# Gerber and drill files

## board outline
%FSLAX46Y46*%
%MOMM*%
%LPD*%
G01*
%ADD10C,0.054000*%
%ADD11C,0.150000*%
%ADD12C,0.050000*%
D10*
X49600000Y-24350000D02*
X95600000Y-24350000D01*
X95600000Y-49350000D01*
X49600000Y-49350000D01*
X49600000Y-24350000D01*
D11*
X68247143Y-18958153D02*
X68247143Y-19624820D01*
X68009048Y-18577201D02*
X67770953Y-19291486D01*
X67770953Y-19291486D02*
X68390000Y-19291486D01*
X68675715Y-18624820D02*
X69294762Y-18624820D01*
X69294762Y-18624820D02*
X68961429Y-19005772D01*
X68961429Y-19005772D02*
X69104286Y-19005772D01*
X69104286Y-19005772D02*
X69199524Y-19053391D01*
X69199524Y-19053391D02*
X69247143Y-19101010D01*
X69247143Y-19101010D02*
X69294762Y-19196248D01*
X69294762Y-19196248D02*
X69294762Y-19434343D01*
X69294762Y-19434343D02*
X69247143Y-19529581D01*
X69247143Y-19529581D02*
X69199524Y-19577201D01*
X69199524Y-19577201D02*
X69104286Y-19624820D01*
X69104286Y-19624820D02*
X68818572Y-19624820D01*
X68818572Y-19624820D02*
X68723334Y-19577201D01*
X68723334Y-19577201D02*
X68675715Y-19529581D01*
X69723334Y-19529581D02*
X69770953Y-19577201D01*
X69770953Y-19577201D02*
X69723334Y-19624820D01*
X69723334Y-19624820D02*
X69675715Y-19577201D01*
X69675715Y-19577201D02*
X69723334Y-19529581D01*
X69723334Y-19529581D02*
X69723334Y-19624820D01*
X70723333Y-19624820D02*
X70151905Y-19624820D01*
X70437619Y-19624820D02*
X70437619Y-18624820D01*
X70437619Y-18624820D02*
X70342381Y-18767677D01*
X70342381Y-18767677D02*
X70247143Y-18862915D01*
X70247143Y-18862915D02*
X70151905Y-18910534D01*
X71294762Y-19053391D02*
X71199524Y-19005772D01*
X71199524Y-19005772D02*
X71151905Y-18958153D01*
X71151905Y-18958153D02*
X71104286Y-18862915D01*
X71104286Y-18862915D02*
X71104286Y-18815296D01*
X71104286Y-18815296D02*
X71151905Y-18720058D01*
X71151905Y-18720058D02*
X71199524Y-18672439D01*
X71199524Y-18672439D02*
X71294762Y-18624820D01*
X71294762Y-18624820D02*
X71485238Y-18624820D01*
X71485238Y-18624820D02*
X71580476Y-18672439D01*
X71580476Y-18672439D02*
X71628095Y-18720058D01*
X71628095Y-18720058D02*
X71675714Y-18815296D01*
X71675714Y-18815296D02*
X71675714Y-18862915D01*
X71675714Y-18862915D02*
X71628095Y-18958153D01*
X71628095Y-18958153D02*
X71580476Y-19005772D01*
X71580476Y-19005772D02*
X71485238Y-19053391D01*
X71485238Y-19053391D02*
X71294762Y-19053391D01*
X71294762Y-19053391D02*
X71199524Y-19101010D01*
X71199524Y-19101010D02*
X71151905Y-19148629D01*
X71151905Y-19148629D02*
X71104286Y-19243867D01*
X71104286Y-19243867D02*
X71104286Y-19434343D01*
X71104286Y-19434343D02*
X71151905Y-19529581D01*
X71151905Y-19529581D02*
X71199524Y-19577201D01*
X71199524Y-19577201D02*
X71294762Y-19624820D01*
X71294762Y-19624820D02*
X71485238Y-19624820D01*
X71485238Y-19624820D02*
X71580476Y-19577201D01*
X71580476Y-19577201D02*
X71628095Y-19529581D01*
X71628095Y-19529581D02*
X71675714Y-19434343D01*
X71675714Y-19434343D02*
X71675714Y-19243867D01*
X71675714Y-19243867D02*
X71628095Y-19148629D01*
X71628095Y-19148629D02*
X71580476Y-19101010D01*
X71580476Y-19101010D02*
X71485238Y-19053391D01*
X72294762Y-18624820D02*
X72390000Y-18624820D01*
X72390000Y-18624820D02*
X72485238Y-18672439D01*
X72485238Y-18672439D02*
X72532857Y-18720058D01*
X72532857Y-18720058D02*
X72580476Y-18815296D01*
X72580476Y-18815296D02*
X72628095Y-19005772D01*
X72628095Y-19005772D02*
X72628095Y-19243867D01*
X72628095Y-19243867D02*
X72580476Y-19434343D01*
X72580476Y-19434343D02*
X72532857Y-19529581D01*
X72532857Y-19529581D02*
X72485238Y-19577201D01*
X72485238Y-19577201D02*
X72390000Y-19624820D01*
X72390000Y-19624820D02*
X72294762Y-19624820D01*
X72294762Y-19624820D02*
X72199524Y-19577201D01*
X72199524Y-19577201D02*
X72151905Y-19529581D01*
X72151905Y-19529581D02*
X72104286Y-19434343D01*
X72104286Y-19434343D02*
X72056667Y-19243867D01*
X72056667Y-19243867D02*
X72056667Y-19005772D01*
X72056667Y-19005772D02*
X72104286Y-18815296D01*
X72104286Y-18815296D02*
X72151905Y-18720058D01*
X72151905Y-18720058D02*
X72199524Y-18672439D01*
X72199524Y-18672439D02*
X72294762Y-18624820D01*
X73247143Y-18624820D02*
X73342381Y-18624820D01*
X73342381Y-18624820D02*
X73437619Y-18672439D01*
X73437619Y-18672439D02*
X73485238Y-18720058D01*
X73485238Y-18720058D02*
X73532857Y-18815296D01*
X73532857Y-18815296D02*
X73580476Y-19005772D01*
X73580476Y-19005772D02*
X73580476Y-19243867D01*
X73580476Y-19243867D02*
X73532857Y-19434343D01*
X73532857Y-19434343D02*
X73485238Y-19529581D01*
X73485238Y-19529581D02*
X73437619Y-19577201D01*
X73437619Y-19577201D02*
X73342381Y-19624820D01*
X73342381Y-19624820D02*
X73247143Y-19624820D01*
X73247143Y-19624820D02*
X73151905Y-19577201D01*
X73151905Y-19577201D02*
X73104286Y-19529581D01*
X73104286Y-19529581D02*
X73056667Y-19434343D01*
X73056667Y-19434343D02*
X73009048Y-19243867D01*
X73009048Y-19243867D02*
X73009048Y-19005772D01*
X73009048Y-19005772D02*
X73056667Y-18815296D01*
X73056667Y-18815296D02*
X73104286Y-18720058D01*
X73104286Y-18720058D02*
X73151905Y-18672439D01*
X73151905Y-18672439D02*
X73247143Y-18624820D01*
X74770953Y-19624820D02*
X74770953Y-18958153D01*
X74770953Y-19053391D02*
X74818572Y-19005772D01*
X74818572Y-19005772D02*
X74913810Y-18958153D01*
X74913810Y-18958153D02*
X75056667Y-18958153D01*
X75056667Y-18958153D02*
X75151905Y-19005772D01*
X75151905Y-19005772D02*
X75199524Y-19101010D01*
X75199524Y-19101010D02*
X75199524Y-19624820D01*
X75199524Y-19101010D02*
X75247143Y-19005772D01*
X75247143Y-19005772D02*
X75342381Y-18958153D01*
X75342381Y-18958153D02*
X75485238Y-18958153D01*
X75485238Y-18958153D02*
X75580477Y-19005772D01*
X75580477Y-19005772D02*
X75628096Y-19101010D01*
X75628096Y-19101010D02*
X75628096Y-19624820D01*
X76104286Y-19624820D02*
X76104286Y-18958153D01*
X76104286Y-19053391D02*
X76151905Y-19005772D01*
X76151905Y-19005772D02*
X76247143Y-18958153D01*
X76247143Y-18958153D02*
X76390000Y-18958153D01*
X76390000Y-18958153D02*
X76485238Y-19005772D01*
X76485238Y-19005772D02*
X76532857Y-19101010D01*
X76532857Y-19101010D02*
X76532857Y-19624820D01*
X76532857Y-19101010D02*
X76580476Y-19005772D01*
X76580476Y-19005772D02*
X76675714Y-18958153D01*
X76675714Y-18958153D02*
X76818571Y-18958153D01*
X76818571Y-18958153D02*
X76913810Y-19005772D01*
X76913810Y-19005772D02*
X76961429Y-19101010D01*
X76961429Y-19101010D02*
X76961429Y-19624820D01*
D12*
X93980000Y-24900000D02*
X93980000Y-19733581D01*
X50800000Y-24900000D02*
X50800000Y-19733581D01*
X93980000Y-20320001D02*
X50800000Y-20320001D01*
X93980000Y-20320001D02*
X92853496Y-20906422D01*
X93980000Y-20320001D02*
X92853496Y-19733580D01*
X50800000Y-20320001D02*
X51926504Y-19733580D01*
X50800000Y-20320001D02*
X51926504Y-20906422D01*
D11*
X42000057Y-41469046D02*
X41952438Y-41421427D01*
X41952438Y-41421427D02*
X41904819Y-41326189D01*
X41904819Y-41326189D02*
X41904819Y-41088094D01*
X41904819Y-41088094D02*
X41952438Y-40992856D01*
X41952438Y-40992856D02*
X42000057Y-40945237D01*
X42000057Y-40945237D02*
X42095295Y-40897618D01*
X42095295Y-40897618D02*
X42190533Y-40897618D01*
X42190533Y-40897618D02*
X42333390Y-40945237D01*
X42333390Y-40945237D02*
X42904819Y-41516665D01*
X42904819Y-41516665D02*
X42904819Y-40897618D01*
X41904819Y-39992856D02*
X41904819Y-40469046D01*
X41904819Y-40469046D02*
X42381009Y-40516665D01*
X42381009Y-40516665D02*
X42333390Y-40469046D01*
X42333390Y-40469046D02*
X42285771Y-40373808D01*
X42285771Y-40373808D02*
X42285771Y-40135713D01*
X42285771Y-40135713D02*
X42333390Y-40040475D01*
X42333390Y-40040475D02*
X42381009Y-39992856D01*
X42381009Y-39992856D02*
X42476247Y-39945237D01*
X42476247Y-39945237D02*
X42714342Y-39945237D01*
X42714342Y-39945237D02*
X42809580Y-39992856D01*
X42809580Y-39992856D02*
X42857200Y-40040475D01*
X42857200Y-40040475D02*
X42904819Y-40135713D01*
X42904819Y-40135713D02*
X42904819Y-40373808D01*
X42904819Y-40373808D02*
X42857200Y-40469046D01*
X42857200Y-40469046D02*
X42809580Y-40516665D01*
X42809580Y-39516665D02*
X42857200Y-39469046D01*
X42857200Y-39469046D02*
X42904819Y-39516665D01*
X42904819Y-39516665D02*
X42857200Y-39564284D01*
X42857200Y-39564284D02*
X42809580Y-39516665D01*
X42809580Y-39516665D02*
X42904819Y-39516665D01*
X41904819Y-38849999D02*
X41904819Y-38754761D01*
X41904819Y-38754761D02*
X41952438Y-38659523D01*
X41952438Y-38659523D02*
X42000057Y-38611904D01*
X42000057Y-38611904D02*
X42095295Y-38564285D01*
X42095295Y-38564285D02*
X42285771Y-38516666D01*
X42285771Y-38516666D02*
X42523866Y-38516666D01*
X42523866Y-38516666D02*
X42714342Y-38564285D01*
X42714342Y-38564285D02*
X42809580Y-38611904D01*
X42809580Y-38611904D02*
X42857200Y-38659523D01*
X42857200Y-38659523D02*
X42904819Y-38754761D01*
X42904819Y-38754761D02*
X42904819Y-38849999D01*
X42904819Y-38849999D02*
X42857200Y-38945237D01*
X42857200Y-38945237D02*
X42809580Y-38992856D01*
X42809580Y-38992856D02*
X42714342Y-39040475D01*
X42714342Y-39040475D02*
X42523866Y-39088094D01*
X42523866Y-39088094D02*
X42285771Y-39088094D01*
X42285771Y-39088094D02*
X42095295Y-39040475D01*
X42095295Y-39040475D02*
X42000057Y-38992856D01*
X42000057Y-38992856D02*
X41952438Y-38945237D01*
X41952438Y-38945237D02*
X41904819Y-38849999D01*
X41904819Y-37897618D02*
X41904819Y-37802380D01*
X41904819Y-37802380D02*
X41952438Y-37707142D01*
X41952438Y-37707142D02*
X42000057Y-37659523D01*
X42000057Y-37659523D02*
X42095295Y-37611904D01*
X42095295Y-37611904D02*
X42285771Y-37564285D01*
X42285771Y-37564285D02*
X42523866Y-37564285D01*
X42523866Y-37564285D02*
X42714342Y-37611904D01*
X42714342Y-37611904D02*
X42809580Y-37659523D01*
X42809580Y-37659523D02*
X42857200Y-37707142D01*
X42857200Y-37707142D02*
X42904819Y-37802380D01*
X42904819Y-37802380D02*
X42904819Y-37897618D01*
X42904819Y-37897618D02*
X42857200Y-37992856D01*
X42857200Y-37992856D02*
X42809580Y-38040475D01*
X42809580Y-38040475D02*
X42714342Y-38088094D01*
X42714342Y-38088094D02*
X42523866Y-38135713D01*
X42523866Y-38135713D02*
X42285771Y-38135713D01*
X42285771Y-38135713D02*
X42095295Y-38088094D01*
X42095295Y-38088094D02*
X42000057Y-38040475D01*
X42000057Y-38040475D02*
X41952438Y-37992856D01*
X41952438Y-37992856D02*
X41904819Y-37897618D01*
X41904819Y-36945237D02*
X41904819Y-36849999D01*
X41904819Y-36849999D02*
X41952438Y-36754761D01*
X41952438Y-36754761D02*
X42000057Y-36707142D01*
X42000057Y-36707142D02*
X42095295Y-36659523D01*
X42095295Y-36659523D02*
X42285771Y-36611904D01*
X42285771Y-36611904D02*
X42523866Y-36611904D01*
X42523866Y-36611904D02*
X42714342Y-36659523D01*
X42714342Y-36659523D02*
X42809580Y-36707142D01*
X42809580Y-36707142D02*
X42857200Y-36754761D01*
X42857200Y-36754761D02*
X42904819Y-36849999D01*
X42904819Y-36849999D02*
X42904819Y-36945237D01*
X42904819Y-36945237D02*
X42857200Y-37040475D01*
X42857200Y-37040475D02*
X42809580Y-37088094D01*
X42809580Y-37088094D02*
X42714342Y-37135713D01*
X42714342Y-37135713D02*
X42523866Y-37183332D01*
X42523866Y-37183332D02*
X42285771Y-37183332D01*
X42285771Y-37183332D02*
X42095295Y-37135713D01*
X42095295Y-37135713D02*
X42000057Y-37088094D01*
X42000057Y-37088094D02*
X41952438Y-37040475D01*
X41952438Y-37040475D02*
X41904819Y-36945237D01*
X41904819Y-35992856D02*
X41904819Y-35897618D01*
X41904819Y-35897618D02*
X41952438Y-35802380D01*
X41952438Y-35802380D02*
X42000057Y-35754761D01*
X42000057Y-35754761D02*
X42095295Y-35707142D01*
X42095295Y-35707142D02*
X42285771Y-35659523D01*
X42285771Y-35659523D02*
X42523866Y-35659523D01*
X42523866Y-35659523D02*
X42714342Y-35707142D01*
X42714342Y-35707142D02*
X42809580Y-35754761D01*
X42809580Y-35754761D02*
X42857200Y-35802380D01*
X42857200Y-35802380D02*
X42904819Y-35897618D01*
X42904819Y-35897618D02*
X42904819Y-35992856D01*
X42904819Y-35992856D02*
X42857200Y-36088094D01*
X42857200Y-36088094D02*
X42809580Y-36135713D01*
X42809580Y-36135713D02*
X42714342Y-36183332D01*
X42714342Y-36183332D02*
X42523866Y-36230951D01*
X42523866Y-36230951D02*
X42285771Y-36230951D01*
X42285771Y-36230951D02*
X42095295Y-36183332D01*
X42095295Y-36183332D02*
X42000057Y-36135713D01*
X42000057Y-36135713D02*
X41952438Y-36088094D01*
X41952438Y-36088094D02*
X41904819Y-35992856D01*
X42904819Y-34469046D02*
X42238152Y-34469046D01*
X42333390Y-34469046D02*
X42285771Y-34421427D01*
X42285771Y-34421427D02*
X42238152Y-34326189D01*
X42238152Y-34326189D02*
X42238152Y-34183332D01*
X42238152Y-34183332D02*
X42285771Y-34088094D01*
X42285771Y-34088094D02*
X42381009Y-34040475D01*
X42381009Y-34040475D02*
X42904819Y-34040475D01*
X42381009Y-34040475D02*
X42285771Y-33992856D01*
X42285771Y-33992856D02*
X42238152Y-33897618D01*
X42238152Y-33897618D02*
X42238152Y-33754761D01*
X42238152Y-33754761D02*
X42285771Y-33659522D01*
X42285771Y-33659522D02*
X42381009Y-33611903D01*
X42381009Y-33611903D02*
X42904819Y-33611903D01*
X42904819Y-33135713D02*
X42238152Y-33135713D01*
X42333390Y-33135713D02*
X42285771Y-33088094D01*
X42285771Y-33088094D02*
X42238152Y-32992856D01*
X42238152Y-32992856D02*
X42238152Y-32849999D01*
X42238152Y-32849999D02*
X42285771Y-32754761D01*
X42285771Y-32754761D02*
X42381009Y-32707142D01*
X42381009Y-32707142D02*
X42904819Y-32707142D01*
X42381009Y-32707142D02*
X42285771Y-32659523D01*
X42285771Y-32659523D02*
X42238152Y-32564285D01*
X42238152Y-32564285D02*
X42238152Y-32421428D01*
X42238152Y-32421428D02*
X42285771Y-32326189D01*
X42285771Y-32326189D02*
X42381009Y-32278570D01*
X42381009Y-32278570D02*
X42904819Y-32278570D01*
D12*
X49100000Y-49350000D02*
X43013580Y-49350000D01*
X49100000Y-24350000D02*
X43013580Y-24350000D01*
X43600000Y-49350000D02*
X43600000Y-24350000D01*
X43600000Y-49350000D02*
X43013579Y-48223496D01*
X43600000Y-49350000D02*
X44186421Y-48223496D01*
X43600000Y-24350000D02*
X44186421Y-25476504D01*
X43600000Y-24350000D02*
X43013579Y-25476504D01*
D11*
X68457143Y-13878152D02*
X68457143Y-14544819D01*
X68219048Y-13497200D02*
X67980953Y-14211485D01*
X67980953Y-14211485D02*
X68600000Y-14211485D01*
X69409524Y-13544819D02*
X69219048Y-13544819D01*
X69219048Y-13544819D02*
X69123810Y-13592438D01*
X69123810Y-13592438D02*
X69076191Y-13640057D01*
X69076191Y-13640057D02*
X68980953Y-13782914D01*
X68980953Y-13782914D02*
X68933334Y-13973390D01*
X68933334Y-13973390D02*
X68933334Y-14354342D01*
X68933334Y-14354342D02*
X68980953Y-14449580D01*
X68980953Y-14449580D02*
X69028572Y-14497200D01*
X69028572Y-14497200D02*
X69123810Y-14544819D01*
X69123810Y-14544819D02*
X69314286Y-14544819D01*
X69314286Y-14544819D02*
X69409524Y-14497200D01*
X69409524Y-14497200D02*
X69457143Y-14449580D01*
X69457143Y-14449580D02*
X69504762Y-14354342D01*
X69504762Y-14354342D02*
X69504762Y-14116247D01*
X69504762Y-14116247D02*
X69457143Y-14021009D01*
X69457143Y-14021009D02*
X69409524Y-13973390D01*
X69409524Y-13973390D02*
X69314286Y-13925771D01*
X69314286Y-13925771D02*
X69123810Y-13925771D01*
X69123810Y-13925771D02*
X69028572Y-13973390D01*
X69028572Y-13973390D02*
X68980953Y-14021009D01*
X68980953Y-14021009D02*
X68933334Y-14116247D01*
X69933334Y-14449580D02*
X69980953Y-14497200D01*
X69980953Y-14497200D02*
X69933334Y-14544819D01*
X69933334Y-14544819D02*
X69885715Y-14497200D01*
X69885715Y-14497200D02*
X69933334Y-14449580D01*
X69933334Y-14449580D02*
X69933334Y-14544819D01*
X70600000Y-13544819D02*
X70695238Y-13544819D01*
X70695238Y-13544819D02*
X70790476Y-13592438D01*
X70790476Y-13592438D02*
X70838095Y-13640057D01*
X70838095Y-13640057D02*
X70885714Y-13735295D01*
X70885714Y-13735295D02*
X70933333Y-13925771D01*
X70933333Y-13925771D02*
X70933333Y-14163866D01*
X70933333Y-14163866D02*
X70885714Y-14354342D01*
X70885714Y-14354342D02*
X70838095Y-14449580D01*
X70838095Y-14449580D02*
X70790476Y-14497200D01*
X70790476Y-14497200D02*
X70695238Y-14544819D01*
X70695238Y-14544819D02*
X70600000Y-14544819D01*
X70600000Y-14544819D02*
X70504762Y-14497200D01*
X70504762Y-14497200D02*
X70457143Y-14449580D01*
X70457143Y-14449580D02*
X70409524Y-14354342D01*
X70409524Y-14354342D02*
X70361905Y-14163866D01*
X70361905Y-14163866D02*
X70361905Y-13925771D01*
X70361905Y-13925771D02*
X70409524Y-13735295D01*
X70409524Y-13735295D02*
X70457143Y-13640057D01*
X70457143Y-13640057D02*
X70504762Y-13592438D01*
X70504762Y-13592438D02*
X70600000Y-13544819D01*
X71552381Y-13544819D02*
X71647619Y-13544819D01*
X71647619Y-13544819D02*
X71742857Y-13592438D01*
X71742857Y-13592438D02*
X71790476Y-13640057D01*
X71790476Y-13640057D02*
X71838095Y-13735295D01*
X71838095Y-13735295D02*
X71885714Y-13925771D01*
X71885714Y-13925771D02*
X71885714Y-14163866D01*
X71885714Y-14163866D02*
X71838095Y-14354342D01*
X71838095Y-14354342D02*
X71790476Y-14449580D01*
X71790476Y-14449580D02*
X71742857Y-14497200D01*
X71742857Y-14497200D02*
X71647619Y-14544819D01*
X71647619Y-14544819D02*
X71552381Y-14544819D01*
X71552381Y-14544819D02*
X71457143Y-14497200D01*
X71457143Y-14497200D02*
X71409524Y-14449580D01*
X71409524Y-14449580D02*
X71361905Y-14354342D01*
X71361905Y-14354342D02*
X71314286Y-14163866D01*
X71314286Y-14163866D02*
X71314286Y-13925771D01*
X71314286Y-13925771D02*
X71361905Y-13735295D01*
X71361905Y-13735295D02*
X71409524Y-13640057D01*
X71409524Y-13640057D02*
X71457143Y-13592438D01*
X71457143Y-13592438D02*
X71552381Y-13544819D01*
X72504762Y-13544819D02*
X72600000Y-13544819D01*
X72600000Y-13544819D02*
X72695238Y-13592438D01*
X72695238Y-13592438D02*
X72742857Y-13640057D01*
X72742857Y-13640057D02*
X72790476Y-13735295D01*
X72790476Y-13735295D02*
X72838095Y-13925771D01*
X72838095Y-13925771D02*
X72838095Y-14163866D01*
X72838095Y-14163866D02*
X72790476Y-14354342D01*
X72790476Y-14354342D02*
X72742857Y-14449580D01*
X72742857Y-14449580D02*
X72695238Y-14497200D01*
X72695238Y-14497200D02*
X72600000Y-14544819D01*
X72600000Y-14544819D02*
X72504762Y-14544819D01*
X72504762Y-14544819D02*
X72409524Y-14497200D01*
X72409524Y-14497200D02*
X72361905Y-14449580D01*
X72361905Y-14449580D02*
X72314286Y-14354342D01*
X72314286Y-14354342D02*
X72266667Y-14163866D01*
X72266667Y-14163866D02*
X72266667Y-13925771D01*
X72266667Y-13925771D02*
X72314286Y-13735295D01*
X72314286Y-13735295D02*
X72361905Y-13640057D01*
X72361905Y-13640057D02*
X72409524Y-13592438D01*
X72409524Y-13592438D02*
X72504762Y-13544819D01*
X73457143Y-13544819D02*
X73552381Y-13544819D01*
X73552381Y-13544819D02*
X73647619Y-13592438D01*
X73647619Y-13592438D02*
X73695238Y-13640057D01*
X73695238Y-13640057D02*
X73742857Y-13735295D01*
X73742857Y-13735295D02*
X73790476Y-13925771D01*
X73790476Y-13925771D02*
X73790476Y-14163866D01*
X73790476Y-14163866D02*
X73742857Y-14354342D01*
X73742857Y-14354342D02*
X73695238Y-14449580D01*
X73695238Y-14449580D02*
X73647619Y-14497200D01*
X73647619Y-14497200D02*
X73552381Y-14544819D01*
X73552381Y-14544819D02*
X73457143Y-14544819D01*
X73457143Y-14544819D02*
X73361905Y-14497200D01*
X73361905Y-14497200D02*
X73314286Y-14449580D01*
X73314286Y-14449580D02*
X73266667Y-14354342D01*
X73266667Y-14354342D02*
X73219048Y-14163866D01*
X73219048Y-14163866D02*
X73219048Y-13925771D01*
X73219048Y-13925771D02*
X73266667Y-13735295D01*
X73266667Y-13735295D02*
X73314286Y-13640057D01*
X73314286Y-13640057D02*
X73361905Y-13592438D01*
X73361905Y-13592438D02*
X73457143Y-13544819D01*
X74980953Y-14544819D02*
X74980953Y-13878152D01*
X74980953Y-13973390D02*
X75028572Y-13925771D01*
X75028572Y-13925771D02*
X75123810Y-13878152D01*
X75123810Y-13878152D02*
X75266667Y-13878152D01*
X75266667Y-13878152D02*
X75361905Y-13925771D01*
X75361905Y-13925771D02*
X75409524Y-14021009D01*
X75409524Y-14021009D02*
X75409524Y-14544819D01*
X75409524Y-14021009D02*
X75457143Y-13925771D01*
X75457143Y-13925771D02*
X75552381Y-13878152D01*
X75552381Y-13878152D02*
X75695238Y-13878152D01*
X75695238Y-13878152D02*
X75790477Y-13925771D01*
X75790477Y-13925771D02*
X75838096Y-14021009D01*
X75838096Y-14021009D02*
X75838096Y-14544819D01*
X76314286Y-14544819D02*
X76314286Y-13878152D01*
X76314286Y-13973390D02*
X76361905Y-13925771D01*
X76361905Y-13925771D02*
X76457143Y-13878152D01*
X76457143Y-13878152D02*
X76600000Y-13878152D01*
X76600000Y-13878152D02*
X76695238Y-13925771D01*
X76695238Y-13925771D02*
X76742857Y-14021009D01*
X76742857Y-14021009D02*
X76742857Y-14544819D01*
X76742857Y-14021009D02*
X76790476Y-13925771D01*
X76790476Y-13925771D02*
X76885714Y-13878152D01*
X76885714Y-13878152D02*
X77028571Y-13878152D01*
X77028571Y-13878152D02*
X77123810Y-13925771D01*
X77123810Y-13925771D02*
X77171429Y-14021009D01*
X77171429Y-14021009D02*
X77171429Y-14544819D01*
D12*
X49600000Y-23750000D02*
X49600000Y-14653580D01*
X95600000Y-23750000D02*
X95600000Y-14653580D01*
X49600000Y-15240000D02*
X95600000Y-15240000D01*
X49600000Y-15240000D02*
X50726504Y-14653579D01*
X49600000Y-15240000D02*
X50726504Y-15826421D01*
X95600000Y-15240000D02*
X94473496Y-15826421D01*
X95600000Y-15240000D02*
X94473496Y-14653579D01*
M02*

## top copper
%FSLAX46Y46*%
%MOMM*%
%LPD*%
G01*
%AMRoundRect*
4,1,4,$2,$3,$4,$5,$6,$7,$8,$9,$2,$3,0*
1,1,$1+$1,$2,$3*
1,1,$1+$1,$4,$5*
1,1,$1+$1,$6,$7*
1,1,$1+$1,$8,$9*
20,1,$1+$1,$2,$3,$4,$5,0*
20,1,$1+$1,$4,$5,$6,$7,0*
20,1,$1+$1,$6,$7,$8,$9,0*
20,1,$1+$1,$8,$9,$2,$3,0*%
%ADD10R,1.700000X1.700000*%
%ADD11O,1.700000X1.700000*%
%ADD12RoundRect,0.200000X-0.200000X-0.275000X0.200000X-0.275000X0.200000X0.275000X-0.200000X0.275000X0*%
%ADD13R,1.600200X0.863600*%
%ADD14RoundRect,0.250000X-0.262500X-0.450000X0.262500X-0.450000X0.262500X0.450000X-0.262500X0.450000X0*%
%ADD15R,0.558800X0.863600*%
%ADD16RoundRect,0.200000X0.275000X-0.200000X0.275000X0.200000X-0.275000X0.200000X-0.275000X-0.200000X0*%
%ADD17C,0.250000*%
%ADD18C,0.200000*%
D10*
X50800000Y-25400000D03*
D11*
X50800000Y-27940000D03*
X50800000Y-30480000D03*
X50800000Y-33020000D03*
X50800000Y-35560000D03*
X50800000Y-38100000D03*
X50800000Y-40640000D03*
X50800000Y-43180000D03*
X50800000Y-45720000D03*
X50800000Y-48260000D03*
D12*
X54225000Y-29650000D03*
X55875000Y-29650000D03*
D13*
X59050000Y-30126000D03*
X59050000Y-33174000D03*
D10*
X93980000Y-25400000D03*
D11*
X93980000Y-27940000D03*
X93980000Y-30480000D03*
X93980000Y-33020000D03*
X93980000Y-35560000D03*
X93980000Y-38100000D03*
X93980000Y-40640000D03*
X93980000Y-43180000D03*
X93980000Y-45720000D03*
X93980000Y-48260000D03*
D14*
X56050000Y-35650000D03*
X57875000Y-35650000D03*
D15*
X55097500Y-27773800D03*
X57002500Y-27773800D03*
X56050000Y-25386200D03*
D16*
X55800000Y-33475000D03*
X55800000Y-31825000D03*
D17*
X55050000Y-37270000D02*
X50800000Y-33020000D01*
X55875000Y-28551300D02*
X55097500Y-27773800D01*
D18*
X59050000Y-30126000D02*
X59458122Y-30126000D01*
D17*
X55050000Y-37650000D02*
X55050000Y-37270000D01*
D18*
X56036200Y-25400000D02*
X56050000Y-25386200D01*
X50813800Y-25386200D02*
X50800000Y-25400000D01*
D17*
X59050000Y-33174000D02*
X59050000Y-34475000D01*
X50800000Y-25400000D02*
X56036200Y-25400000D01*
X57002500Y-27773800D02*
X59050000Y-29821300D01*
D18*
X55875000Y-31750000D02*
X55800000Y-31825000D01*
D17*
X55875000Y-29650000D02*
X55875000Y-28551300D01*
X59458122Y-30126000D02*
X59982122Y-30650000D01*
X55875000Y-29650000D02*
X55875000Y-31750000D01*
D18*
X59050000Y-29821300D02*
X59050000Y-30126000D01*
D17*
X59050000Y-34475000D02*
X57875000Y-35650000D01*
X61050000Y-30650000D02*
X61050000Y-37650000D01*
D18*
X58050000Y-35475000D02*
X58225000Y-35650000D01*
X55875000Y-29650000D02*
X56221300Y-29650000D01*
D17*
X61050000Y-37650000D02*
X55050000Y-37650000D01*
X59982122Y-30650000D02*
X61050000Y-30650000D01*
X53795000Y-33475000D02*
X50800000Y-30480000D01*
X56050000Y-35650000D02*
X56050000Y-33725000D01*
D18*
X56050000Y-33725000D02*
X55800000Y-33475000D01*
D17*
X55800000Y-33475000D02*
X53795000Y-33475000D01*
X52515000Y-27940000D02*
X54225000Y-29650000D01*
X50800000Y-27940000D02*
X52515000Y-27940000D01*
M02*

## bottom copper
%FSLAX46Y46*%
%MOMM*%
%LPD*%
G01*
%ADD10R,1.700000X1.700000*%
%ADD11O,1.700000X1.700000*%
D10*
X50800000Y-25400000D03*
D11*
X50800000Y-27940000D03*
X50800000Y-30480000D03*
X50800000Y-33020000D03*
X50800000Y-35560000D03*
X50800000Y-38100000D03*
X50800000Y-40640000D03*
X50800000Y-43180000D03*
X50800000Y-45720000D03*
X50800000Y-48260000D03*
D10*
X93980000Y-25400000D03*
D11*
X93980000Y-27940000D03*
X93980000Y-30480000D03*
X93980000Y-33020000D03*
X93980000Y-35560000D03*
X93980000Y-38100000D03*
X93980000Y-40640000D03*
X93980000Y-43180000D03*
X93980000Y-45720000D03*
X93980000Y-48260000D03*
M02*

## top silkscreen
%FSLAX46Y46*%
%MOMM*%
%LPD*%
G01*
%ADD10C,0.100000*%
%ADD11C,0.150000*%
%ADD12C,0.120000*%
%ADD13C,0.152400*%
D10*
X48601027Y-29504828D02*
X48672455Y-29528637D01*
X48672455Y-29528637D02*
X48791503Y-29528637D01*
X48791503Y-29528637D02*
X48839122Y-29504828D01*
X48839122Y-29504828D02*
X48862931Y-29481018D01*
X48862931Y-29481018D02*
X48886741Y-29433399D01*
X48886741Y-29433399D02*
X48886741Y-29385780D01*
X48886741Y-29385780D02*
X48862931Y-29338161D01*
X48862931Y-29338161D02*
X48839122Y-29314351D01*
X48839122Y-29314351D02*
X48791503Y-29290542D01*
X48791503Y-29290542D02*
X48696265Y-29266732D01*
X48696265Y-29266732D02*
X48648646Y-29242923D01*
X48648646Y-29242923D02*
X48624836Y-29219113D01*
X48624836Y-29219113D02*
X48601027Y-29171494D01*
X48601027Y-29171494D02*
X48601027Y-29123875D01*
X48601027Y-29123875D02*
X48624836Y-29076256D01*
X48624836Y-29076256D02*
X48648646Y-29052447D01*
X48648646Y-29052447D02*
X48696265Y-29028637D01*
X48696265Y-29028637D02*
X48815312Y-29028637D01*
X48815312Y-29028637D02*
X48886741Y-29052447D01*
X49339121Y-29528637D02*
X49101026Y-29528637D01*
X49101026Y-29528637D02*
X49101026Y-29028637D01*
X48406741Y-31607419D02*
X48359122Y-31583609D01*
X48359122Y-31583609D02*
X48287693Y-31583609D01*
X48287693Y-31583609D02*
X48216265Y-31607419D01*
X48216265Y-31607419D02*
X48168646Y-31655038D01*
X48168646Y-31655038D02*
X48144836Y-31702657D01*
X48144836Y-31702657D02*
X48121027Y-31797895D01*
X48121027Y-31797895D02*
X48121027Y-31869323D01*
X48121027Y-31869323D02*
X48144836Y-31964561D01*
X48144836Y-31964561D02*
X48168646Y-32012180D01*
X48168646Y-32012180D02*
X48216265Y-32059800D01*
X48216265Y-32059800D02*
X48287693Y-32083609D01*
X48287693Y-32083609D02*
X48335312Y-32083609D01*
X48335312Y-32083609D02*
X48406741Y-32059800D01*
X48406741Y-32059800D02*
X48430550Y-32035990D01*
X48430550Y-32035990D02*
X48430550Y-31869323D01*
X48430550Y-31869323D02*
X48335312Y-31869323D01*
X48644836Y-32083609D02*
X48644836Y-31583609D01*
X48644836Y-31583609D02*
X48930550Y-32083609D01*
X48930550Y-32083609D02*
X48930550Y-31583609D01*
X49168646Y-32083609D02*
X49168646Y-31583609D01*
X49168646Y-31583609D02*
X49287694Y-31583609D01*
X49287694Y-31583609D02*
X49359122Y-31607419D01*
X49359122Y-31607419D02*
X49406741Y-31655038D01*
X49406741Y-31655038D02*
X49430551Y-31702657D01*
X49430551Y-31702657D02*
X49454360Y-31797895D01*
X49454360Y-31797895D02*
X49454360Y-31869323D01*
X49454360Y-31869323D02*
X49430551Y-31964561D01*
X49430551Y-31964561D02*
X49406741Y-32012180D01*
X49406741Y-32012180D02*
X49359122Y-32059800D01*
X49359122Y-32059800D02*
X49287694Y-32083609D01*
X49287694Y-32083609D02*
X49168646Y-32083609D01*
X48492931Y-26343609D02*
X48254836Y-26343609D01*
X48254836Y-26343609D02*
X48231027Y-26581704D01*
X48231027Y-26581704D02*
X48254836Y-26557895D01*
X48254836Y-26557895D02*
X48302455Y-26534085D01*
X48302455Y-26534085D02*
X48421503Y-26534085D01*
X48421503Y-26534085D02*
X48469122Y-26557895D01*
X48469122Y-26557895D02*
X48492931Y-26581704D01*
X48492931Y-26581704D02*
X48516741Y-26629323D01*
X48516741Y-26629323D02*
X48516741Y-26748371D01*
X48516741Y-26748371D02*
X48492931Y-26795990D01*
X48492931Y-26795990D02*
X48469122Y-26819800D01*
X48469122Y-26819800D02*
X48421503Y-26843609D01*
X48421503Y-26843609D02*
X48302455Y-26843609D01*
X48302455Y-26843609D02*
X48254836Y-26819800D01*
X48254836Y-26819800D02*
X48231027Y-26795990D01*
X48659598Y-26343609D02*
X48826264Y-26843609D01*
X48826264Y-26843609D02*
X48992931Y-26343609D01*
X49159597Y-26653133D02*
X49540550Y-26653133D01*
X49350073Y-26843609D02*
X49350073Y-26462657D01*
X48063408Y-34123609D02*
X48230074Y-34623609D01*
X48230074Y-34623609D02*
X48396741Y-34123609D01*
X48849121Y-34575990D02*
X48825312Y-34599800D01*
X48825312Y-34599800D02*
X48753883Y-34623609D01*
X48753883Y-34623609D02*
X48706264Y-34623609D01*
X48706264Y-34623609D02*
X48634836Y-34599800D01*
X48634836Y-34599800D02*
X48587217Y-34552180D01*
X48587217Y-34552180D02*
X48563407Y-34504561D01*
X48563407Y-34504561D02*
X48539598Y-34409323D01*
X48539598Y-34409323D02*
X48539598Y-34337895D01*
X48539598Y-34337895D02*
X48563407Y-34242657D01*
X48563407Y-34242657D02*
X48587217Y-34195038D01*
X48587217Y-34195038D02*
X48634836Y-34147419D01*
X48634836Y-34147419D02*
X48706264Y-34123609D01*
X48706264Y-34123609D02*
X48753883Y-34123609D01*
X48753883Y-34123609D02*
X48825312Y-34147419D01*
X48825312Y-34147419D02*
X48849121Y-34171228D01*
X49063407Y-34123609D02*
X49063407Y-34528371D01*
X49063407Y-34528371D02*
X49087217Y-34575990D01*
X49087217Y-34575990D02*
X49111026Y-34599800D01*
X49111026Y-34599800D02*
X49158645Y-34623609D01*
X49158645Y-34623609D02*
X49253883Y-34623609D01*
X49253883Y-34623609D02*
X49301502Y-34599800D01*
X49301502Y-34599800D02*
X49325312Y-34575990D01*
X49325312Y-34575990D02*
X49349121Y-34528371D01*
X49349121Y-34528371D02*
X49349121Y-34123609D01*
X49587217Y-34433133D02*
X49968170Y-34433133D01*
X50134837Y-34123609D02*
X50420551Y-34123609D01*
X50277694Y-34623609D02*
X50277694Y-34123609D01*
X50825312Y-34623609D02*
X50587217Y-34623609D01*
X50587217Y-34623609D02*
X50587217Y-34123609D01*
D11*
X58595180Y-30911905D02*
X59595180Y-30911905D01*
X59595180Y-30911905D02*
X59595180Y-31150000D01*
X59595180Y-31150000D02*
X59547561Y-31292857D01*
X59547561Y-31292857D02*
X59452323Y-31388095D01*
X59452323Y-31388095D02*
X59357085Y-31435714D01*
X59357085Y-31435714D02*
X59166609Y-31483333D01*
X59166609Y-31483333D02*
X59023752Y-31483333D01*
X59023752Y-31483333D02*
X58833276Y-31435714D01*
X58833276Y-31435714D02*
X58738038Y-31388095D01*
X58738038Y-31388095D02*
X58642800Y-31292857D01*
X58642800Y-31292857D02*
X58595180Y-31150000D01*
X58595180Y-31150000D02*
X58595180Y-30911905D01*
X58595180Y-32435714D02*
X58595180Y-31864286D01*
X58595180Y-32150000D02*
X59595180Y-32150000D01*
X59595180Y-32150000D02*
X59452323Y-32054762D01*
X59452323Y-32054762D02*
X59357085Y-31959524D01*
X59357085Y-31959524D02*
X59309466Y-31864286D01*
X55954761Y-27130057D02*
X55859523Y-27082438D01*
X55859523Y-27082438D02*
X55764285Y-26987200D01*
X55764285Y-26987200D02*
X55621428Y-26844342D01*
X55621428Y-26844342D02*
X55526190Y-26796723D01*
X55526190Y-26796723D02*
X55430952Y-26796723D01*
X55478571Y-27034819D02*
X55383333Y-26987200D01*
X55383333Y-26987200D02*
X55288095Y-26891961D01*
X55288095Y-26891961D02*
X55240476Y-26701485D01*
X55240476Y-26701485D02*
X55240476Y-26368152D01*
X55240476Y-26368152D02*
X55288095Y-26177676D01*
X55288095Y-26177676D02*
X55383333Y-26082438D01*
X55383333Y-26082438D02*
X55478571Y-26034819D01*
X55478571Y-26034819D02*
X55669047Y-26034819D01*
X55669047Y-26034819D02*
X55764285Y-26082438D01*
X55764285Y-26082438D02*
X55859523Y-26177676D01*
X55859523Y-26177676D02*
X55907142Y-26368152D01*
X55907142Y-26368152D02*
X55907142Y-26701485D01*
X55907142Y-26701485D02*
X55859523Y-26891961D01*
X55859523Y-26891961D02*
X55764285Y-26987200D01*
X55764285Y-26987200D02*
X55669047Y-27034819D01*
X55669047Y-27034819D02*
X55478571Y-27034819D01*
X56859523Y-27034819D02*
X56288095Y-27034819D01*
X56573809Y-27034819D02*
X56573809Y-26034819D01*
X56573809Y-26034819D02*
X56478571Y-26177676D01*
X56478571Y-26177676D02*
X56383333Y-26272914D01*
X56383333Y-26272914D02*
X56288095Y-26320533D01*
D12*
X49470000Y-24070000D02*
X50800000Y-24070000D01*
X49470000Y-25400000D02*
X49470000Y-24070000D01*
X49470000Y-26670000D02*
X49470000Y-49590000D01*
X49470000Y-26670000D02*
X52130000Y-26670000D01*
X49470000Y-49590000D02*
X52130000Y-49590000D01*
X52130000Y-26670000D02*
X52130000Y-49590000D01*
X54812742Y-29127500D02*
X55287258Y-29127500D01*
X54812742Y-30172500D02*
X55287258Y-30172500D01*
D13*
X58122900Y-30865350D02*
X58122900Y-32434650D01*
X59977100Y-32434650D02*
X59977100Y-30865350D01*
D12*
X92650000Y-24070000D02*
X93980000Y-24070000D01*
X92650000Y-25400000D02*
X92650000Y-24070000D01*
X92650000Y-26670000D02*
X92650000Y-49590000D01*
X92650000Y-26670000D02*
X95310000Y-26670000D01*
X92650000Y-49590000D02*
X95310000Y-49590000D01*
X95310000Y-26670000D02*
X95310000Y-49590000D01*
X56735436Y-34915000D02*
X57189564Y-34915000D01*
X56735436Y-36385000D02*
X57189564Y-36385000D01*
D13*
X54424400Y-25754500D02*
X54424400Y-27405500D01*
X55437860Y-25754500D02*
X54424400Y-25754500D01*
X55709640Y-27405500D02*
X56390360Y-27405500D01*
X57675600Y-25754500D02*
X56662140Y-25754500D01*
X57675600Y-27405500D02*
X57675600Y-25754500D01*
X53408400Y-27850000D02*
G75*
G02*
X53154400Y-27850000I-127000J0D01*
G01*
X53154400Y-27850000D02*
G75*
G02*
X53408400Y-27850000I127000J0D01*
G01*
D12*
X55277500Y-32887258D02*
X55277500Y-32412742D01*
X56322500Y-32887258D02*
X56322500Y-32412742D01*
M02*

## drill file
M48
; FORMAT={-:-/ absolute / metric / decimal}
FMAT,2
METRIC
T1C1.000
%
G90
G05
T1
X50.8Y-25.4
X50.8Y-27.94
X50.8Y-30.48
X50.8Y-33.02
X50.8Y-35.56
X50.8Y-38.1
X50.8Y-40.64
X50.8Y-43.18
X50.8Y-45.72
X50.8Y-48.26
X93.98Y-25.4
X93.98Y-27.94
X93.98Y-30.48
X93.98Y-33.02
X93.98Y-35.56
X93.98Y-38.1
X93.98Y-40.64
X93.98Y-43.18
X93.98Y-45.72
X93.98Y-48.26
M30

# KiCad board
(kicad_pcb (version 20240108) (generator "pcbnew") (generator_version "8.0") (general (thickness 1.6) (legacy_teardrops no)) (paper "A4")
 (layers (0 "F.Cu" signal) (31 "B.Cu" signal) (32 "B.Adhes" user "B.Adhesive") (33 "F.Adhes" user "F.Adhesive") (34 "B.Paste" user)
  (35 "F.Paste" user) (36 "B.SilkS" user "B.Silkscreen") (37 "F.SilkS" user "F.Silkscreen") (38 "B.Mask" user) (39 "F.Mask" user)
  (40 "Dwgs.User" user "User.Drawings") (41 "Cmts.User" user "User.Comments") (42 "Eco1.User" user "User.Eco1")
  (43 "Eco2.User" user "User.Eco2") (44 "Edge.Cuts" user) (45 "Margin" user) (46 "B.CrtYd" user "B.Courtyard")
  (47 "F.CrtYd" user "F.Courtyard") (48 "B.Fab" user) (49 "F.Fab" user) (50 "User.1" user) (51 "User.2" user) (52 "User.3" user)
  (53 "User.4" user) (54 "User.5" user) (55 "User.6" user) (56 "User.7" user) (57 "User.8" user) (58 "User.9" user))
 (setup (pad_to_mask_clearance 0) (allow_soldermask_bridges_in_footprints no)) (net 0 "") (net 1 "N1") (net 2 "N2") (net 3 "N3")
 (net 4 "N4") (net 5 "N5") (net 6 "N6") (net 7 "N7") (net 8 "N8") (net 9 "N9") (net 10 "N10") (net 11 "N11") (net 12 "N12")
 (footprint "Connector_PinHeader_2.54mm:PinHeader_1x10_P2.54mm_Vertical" (layer "F.Cu") (at 50.8 25.4)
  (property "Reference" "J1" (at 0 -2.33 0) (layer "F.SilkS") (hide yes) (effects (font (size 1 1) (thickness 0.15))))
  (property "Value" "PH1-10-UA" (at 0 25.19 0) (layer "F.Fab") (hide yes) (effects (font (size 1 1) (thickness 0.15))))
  (fp_line (start -1.33 -1.33) (end 0 -1.33) (stroke (width 0.12) (type solid)) (layer "F.SilkS"))
  (fp_line (start -1.33 0) (end -1.33 -1.33) (stroke (width 0.12) (type solid)) (layer "F.SilkS"))
  (fp_line (start -1.33 1.27) (end -1.33 24.19) (stroke (width 0.12) (type solid)) (layer "F.SilkS"))
  (fp_line (start -1.33 1.27) (end 1.33 1.27) (stroke (width 0.12) (type solid)) (layer "F.SilkS"))
  (fp_line (start -1.33 24.19) (end 1.33 24.19) (stroke (width 0.12) (type solid)) (layer "F.SilkS"))
  (fp_line (start 1.33 1.27) (end 1.33 24.19) (stroke (width 0.12) (type solid)) (layer "F.SilkS"))
  (pad "1" thru_hole rect (at 0 0) (size 1.7 1.7) (drill 1) (layers "*.Cu" "*.Mask") (remove_unused_layers no) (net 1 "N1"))
  (pad "2" thru_hole oval (at 0 2.54) (size 1.7 1.7) (drill 1) (layers "*.Cu" "*.Mask") (remove_unused_layers no) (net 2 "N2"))
  (pad "3" thru_hole oval (at 0 5.08) (size 1.7 1.7) (drill 1) (layers "*.Cu" "*.Mask") (remove_unused_layers no) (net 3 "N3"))
  (pad "4" thru_hole oval (at 0 7.62) (size 1.7 1.7) (drill 1) (layers "*.Cu" "*.Mask") (remove_unused_layers no) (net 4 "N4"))
  (pad "5" thru_hole oval (at 0 10.16) (size 1.7 1.7) (drill 1) (layers "*.Cu" "*.Mask") (remove_unused_layers no) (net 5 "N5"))
  (pad "6" thru_hole oval (at 0 12.7) (size 1.7 1.7) (drill 1) (layers "*.Cu" "*.Mask") (remove_unused_layers no) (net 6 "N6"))
  (pad "7" thru_hole oval (at 0 15.24) (size 1.7 1.7) (drill 1) (layers "*.Cu" "*.Mask") (remove_unused_layers no) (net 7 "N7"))
  (pad "8" thru_hole oval (at 0 17.78) (size 1.7 1.7) (drill 1) (layers "*.Cu" "*.Mask") (remove_unused_layers no) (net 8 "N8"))
  (pad "9" thru_hole oval (at 0 20.32) (size 1.7 1.7) (drill 1) (layers "*.Cu" "*.Mask") (remove_unused_layers no) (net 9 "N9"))
  (pad "10" thru_hole oval (at 0 22.86) (size 1.7 1.7) (drill 1) (layers "*.Cu" "*.Mask") (remove_unused_layers no) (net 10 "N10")))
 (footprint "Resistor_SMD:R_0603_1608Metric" (layer "F.Cu") (at 55.05 29.65)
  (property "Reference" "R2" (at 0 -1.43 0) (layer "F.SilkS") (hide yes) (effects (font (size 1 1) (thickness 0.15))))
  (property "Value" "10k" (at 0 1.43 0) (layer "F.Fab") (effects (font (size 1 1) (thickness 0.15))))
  (fp_line (start -0.237258 -0.5225) (end 0.237258 -0.5225) (stroke (width 0.12) (type solid)) (layer "F.SilkS"))
  (fp_line (start -0.237258 0.5225) (end 0.237258 0.5225) (stroke (width 0.12) (type solid)) (layer "F.SilkS"))
  (pad "1" smd roundrect (at -0.825 0) (size 0.8 0.95) (layers "F.Cu" "F.Paste" "F.Mask") (roundrect_rratio 0.25) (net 2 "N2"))
  (pad "2" smd roundrect (at 0.825 0) (size 0.8 0.95) (layers "F.Cu" "F.Paste" "F.Mask") (roundrect_rratio 0.25) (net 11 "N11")))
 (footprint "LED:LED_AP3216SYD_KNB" (layer "F.Cu") (at 59.05 31.65 -90)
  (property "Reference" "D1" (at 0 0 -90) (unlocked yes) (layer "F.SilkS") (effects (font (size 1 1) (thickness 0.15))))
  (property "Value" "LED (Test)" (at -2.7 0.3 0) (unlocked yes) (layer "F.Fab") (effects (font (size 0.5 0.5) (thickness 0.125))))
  (fp_line (start -0.78465 0.9271) (end 0.78465 0.9271) (stroke (width 0.1524) (type solid)) (layer "F.SilkS"))
  (fp_line (start 0.78465 -0.9271) (end -0.78465 -0.9271) (stroke (width 0.1524) (type solid)) (layer "F.SilkS"))
  (pad "1" smd rect (at -1.524 0 270) (size 0.8636 1.6002) (layers "F.Cu" "F.Paste" "F.Mask") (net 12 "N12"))
  (pad "2" smd rect (at 1.524 0 270) (size 0.8636 1.6002) (layers "F.Cu" "F.Paste" "F.Mask") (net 4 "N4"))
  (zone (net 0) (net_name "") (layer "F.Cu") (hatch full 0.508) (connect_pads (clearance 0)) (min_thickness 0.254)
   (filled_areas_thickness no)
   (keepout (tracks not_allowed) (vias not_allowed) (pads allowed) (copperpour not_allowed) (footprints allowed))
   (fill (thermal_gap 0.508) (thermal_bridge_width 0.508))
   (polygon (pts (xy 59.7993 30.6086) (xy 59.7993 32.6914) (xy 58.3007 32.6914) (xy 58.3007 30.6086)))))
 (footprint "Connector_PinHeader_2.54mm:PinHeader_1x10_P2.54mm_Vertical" (layer "F.Cu") (at 93.98 25.4)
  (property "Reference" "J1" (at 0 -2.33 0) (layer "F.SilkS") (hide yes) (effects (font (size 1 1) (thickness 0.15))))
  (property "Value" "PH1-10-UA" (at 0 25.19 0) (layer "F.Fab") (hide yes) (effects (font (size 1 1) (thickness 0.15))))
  (fp_line (start -1.33 -1.33) (end 0 -1.33) (stroke (width 0.12) (type solid)) (layer "F.SilkS"))
  (fp_line (start -1.33 0) (end -1.33 -1.33) (stroke (width 0.12) (type solid)) (layer "F.SilkS"))
  (fp_line (start -1.33 1.27) (end -1.33 24.19) (stroke (width 0.12) (type solid)) (layer "F.SilkS"))
  (fp_line (start -1.33 1.27) (end 1.33 1.27) (stroke (width 0.12) (type solid)) (layer "F.SilkS"))
  (fp_line (start -1.33 24.19) (end 1.33 24.19) (stroke (width 0.12) (type solid)) (layer "F.SilkS"))
  (fp_line (start 1.33 1.27) (end 1.33 24.19) (stroke (width 0.12) (type solid)) (layer "F.SilkS"))
  (pad "1" thru_hole rect (at 0 0) (size 1.7 1.7) (drill 1) (layers "*.Cu" "*.Mask") (remove_unused_layers no))
  (pad "2" thru_hole oval (at 0 2.54) (size 1.7 1.7) (drill 1) (layers "*.Cu" "*.Mask") (remove_unused_layers no))
  (pad "3" thru_hole oval (at 0 5.08) (size 1.7 1.7) (drill 1) (layers "*.Cu" "*.Mask") (remove_unused_layers no))
  (pad "4" thru_hole oval (at 0 7.62) (size 1.7 1.7) (drill 1) (layers "*.Cu" "*.Mask") (remove_unused_layers no))
  (pad "5" thru_hole oval (at 0 10.16) (size 1.7 1.7) (drill 1) (layers "*.Cu" "*.Mask") (remove_unused_layers no))
  (pad "6" thru_hole oval (at 0 12.7) (size 1.7 1.7) (drill 1) (layers "*.Cu" "*.Mask") (remove_unused_layers no))
  (pad "7" thru_hole oval (at 0 15.24) (size 1.7 1.7) (drill 1) (layers "*.Cu" "*.Mask") (remove_unused_layers no))
  (pad "8" thru_hole oval (at 0 17.78) (size 1.7 1.7) (drill 1) (layers "*.Cu" "*.Mask") (remove_unused_layers no))
  (pad "9" thru_hole oval (at 0 20.32) (size 1.7 1.7) (drill 1) (layers "*.Cu" "*.Mask") (remove_unused_layers no))
  (pad "10" thru_hole oval (at 0 22.86) (size 1.7 1.7) (drill 1) (layers "*.Cu" "*.Mask") (remove_unused_layers no)))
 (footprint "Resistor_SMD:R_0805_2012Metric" (layer "F.Cu") (at 56.9625 35.65)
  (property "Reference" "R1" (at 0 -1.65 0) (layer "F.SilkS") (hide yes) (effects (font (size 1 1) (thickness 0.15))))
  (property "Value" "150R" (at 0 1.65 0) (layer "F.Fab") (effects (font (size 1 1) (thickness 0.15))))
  (fp_line (start -0.227064 -0.735) (end 0.227064 -0.735) (stroke (width 0.12) (type solid)) (layer "F.SilkS"))
  (fp_line (start -0.227064 0.735) (end 0.227064 0.735) (stroke (width 0.12) (type solid)) (layer "F.SilkS"))
  (pad "1" smd roundrect (at -0.9125 0) (size 1.025 1.4) (layers "F.Cu" "F.Paste" "F.Mask") (roundrect_rratio 0.243902) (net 3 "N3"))
  (pad "2" smd roundrect (at 0.9125 0) (size 1.025 1.4) (layers "F.Cu" "F.Paste" "F.Mask") (roundrect_rratio 0.243902) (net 12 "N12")))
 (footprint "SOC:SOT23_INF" (layer "F.Cu") (at 56.05 26.58)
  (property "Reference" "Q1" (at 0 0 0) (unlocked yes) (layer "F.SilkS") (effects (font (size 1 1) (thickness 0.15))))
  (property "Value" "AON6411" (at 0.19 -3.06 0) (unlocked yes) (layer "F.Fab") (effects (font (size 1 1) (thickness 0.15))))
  (fp_line (start -1.6256 -0.8255) (end -1.6256 0.8255) (stroke (width 0.1524) (type solid)) (layer "F.SilkS"))
  (fp_line (start -0.61214 -0.8255) (end -1.6256 -0.8255) (stroke (width 0.1524) (type solid)) (layer "F.SilkS"))
  (fp_line (start -0.34036 0.8255) (end 0.34036 0.8255) (stroke (width 0.1524) (type solid)) (layer "F.SilkS"))
  (fp_line (start 1.6256 -0.8255) (end 0.61214 -0.8255) (stroke (width 0.1524) (type solid)) (layer "F.SilkS"))
  (fp_line (start 1.6256 0.8255) (end 1.6256 -0.8255) (stroke (width 0.1524) (type solid)) (layer "F.SilkS"))
  (fp_circle (center -2.7686 1.27) (end -2.6416 1.27) (stroke (width 0.1524) (type solid)) (fill none) (layer "F.SilkS"))
  (pad "1" smd rect (at -0.9525 1.1938) (size 0.5588 0.8636) (layers "F.Cu" "F.Paste" "F.Mask") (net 4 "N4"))
  (pad "2" smd rect (at 0.9525 1.1938) (size 0.5588 0.8636) (layers "F.Cu" "F.Paste" "F.Mask") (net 4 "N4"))
  (pad "3" smd rect (at 0 -1.1938) (size 0.5588 0.8636) (layers "F.Cu" "F.Paste" "F.Mask") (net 4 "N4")))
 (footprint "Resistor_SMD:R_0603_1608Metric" (layer "F.Cu") (at 55.8 32.65 90)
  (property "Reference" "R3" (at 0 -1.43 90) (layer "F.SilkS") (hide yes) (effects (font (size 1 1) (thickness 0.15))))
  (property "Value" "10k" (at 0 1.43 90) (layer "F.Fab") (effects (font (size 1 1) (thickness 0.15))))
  (fp_line (start -0.237258 -0.5225) (end 0.237258 -0.5225) (stroke (width 0.12) (type solid)) (layer "F.SilkS"))
  (fp_line (start -0.237258 0.5225) (end 0.237258 0.5225) (stroke (width 0.12) (type solid)) (layer "F.SilkS"))
  (pad "1" smd roundrect (at -0.825 0 90) (size 0.8 0.95) (layers "F.Cu" "F.Paste" "F.Mask") (roundrect_rratio 0.25) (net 3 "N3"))
  (pad "2" smd roundrect (at 0.825 0 90) (size 0.8 0.95) (layers "F.Cu" "F.Paste" "F.Mask") (roundrect_rratio 0.25) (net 11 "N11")))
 (gr_rect (start 49.6 24.35) (end 95.6 49.35) (stroke (width 0.054) (type default)) (fill none) (layer "Edge.Cuts"))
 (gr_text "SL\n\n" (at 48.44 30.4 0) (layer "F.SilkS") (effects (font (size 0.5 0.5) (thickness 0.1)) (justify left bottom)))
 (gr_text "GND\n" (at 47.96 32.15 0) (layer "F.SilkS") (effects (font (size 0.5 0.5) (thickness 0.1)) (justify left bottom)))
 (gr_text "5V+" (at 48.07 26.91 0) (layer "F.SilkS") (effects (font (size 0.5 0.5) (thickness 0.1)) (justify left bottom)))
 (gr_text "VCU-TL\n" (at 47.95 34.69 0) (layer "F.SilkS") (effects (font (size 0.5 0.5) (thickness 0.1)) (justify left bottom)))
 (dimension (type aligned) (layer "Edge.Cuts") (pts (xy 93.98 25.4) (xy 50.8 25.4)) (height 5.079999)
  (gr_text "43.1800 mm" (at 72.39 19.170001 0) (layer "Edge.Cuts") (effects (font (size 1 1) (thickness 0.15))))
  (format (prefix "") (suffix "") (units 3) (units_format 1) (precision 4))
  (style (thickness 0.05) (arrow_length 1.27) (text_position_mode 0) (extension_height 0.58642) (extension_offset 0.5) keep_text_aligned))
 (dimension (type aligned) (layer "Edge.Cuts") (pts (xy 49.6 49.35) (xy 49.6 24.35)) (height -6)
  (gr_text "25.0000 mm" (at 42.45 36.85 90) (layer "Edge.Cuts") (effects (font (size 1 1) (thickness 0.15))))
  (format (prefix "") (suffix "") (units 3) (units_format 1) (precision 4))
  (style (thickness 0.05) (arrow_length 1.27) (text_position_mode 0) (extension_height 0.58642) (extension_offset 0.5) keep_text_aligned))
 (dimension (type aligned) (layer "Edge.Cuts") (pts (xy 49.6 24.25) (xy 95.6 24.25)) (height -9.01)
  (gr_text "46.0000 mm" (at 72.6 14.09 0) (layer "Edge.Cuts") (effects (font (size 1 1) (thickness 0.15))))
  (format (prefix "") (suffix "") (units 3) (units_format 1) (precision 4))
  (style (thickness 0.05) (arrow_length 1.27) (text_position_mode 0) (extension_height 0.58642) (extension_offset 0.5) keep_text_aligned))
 (segment (start 55.05 37.27) (end 50.8 33.02) (width 0.25) (layer "F.Cu") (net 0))
 (segment (start 55.875 28.5513) (end 55.0975 27.7738) (width 0.25) (layer "F.Cu") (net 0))
 (segment (start 59.05 30.126) (end 59.458122 30.126) (width 0.2) (layer "F.Cu") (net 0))
 (segment (start 55.05 37.65) (end 55.05 37.27) (width 0.25) (layer "F.Cu") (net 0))
 (segment (start 56.0362 25.4) (end 56.05 25.3862) (width 0.2) (layer "F.Cu") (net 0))
 (segment (start 50.8138 25.3862) (end 50.8 25.4) (width 0.2) (layer "F.Cu") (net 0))
 (segment (start 59.05 33.174) (end 59.05 34.475) (width 0.25) (layer "F.Cu") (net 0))
 (segment (start 50.8 25.4) (end 56.0362 25.4) (width 0.25) (layer "F.Cu") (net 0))
 (segment (start 57.0025 27.7738) (end 59.05 29.8213) (width 0.25) (layer "F.Cu") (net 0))
 (segment (start 55.875 31.75) (end 55.8 31.825) (width 0.2) (layer "F.Cu") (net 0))
 (segment (start 55.875 29.65) (end 55.875 28.5513) (width 0.25) (layer "F.Cu") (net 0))
 (segment (start 59.458122 30.126) (end 59.982122 30.65) (width 0.25) (layer "F.Cu") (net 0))
 (segment (start 55.875 29.65) (end 55.875 31.75) (width 0.25) (layer "F.Cu") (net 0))
 (segment (start 59.05 29.8213) (end 59.05 30.126) (width 0.2) (layer "F.Cu") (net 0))
 (segment (start 59.05 34.475) (end 57.875 35.65) (width 0.25) (layer "F.Cu") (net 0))
 (segment (start 61.05 30.65) (end 61.05 37.65) (width 0.25) (layer "F.Cu") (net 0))
 (segment (start 58.05 35.475) (end 58.225 35.65) (width 0.2) (layer "F.Cu") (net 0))
 (segment (start 55.875 29.65) (end 56.2213 29.65) (width 0.2) (layer "F.Cu") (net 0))
 (segment (start 61.05 37.65) (end 55.05 37.65) (width 0.25) (layer "F.Cu") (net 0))
 (segment (start 59.982122 30.65) (end 61.05 30.65) (width 0.25) (layer "F.Cu") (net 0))
 (segment (start 53.795 33.475) (end 50.8 30.48) (width 0.25) (layer "F.Cu") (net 3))
 (segment (start 56.05 35.65) (end 56.05 33.725) (width 0.25) (layer "F.Cu") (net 3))
 (segment (start 56.05 33.725) (end 55.8 33.475) (width 0.2) (layer "F.Cu") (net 3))
 (segment (start 55.8 33.475) (end 53.795 33.475) (width 0.25) (layer "F.Cu") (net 3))
 (segment (start 52.515 27.94) (end 54.225 29.65) (width 0.25) (layer "F.Cu") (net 2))
 (segment (start 50.8 27.94) (end 52.515 27.94) (width 0.25) (layer "F.Cu") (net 2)))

